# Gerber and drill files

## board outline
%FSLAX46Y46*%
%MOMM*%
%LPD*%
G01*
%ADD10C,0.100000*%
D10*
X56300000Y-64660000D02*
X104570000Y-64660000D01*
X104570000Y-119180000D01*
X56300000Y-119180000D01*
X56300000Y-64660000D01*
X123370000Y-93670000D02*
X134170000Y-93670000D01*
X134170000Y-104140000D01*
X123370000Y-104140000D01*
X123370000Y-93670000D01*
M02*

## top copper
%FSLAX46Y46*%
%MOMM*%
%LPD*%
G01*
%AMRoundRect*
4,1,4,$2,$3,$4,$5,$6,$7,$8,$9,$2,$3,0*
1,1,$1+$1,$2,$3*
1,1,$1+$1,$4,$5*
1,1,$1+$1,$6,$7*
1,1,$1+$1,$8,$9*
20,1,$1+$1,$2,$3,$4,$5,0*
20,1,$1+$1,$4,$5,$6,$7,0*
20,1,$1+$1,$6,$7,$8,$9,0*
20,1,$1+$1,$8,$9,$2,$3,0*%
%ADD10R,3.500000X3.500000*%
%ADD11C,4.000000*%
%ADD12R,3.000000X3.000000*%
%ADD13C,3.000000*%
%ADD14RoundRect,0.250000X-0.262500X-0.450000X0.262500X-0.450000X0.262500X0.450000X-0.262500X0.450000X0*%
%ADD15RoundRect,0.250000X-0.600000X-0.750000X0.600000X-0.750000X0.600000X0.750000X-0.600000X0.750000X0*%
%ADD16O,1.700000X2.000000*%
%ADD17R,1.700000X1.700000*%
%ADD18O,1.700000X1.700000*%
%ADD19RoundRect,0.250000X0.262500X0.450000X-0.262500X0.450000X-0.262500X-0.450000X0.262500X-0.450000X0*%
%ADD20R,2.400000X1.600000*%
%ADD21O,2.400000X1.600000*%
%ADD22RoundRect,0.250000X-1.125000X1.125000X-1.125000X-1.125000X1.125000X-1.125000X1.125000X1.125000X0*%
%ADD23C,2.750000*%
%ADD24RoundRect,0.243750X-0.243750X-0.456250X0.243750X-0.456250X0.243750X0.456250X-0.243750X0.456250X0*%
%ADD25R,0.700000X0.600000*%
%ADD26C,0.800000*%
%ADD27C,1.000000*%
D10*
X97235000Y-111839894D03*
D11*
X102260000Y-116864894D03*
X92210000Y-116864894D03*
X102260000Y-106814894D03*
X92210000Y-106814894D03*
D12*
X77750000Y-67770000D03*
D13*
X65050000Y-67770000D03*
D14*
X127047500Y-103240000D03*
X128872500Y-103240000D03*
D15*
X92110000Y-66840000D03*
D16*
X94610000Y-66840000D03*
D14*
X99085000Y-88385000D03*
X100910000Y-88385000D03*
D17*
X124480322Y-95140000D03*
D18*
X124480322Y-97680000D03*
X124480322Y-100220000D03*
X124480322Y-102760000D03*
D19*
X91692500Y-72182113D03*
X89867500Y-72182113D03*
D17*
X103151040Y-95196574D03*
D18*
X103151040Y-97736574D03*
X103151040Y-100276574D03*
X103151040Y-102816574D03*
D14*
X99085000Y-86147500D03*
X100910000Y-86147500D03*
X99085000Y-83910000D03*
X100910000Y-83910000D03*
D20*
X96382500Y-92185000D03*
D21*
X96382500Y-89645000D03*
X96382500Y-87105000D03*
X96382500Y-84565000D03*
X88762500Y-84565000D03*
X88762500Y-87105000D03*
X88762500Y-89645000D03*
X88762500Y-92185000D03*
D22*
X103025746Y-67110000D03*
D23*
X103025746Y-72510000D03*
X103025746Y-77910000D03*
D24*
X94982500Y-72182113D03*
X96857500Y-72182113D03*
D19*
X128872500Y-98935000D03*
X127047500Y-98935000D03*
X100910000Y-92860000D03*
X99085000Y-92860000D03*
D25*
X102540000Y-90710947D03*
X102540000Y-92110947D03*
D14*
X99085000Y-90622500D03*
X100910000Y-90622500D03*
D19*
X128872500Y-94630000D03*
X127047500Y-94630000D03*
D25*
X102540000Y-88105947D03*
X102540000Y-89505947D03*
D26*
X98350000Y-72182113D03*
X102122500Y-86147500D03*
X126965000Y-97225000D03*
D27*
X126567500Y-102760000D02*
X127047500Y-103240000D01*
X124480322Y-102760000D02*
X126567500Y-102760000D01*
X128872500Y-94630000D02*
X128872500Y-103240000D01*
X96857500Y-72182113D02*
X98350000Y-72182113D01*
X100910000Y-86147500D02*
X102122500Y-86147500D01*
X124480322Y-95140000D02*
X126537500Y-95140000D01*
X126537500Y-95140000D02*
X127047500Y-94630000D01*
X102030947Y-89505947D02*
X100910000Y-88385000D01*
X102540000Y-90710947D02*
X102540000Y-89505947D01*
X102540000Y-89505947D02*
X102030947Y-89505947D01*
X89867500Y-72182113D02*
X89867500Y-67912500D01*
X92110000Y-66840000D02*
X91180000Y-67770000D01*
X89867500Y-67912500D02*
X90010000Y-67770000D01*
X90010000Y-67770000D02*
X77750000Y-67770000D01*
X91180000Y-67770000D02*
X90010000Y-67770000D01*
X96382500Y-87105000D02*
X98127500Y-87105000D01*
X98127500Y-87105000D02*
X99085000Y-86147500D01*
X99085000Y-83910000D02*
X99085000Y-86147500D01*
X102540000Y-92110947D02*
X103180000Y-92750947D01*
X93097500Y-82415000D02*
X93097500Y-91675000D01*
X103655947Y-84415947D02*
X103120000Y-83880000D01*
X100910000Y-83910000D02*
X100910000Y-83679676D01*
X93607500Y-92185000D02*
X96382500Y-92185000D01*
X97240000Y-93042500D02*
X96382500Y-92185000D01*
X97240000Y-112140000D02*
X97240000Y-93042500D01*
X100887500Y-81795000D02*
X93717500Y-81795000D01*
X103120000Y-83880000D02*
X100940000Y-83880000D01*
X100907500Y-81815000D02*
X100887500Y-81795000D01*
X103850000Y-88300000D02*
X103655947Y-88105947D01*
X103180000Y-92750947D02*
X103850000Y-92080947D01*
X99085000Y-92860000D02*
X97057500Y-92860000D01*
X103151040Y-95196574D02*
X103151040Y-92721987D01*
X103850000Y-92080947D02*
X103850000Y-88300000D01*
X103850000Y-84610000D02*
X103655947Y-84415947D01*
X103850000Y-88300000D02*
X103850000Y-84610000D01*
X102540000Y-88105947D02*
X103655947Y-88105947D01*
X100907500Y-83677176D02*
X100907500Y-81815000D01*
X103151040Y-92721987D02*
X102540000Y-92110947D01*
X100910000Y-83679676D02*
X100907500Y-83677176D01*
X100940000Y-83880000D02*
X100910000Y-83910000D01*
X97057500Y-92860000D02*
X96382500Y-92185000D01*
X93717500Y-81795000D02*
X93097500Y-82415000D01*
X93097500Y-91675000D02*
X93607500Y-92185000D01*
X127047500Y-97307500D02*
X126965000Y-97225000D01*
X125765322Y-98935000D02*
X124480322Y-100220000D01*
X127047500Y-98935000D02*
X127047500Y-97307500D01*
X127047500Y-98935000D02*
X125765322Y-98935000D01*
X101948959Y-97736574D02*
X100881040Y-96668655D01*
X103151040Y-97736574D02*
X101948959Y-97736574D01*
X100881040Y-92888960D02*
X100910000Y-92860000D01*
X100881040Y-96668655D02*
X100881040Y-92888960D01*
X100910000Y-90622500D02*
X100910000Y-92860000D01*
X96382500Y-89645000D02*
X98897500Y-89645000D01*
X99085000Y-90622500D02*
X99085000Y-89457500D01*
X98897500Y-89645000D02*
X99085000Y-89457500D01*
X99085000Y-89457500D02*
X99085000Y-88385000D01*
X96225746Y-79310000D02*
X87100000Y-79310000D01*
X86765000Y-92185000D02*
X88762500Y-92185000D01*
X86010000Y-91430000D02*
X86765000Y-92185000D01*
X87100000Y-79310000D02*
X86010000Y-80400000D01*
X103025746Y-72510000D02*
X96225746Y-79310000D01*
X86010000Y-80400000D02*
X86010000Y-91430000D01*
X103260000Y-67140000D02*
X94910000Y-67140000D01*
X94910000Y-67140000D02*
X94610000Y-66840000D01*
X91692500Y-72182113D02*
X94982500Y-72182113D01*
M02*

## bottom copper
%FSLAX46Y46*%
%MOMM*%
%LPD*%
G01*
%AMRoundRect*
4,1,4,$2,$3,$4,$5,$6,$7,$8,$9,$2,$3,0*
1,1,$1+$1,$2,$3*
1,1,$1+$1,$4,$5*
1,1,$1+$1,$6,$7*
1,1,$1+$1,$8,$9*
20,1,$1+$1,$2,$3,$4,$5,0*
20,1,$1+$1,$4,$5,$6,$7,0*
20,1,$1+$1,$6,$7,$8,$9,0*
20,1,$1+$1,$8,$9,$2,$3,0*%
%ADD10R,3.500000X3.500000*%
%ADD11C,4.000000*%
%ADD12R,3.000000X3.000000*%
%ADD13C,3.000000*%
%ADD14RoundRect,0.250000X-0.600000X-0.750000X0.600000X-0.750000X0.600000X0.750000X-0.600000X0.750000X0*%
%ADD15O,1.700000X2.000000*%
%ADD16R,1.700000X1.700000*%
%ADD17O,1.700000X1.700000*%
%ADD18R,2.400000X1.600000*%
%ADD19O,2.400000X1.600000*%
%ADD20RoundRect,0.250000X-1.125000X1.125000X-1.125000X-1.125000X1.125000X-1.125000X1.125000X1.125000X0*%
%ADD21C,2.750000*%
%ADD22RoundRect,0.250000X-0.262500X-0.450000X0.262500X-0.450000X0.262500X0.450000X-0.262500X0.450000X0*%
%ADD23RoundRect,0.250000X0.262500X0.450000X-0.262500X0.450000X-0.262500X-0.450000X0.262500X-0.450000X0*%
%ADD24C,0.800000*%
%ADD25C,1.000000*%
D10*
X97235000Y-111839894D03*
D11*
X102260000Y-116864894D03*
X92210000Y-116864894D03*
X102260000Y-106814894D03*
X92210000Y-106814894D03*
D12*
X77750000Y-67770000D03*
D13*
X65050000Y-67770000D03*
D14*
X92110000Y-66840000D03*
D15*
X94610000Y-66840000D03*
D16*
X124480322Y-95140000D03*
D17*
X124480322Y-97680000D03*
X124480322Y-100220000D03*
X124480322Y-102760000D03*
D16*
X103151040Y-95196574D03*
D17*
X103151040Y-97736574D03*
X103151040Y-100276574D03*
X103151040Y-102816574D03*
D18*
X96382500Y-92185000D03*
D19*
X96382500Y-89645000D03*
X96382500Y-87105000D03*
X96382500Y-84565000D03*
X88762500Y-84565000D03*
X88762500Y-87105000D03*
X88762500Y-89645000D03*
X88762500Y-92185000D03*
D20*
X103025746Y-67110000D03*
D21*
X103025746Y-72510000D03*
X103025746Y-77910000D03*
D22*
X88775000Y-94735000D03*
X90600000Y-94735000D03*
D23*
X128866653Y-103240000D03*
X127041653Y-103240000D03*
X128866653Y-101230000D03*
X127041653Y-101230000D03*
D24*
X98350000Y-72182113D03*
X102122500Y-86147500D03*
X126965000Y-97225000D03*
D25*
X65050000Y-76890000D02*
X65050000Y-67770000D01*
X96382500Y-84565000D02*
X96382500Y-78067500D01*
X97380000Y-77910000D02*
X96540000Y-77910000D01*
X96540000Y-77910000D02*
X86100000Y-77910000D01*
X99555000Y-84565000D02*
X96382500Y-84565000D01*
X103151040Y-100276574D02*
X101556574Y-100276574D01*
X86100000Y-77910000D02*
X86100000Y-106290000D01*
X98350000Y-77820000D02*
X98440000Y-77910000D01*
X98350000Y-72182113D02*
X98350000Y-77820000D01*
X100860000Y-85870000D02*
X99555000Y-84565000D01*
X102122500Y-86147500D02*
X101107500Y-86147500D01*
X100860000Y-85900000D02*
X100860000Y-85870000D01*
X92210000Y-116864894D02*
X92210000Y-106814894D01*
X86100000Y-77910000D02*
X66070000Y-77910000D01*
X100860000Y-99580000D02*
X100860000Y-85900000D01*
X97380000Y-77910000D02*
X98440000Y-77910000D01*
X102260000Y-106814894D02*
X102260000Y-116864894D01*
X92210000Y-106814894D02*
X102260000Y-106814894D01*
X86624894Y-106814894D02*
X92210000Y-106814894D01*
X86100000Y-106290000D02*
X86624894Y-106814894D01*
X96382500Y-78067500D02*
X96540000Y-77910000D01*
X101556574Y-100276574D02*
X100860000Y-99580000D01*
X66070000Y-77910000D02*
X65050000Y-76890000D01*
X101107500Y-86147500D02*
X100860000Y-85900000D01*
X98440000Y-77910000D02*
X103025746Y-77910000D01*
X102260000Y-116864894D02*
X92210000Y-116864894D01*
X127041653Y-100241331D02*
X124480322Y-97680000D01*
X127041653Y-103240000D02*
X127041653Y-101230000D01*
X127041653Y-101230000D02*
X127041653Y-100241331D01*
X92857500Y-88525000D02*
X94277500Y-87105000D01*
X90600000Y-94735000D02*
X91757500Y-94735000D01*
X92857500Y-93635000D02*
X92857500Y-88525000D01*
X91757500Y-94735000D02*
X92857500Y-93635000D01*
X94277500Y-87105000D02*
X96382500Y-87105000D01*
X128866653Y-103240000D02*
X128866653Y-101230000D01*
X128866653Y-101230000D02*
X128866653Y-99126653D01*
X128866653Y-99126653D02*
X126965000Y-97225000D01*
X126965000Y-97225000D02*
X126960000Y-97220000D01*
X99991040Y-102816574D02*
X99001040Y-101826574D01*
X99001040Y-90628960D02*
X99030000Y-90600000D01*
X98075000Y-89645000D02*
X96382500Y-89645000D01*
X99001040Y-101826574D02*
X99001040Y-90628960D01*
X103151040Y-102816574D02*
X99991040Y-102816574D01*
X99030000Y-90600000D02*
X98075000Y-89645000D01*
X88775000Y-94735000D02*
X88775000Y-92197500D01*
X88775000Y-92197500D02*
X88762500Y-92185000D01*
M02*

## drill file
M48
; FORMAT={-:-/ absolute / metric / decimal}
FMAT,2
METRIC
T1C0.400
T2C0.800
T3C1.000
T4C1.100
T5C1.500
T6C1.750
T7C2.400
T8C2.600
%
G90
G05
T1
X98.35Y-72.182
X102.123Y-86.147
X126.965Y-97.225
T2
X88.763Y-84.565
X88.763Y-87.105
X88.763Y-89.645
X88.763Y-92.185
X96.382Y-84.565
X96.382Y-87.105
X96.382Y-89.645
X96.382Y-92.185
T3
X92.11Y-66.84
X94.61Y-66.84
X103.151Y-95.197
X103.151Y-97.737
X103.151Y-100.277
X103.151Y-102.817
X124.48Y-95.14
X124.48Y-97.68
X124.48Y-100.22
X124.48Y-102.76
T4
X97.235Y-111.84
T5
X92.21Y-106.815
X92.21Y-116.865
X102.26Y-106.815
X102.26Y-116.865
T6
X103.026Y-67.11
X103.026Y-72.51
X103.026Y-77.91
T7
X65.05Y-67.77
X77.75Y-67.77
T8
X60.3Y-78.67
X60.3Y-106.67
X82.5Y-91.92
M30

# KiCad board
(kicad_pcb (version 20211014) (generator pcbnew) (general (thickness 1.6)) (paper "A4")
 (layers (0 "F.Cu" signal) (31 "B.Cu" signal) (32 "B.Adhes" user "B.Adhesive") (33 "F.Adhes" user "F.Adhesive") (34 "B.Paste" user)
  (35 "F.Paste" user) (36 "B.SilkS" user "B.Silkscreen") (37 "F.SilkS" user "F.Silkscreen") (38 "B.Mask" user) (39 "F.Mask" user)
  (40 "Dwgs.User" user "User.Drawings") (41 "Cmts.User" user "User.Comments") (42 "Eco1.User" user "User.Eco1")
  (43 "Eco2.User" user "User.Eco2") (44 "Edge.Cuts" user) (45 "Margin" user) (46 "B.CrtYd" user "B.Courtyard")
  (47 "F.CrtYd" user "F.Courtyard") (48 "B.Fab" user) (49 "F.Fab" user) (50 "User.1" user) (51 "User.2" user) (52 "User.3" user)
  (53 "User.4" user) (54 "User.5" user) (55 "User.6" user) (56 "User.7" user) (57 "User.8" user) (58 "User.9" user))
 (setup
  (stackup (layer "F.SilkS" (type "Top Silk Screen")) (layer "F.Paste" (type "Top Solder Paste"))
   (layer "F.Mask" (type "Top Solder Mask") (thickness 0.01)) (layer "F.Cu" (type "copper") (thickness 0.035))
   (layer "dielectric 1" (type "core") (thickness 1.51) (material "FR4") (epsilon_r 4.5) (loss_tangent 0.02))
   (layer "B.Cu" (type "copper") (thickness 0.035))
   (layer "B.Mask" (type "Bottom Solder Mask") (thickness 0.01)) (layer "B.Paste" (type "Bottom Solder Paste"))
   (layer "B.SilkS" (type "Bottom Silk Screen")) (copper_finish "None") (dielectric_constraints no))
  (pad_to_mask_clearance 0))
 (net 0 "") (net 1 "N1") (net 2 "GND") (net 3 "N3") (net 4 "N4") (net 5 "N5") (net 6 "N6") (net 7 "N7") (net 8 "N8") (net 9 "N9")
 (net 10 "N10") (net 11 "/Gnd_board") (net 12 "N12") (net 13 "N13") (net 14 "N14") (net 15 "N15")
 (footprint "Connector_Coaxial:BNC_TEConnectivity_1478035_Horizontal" (layer "F.Cu") (at 97.235 111.839894 -90)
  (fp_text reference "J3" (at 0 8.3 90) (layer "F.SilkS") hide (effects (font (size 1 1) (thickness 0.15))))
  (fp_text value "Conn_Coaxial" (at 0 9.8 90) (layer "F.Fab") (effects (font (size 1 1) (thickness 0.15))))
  (pad "1" thru_hole rect (at 0 0 270) (size 3.5 3.5) (drill 1.1) (layers *.Cu *.Mask) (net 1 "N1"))
  (pad "2" thru_hole circle (at 5.025 -5.025 270) (size 4 4) (drill 1.5) (layers *.Cu *.Mask) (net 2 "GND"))
  (pad "2" thru_hole circle (at 5.025 5.025 270) (size 4 4) (drill 1.5) (layers *.Cu *.Mask) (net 2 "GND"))
  (pad "2" thru_hole circle (at -5.025 -5.025 270) (size 4 4) (drill 1.5) (layers *.Cu *.Mask) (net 2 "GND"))
  (pad "2" thru_hole circle (at -5.025 5.025 270) (size 4 4) (drill 1.5) (layers *.Cu *.Mask) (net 2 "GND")))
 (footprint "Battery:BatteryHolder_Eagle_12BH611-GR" (layer "F.Cu") (at 77.75 67.77 90)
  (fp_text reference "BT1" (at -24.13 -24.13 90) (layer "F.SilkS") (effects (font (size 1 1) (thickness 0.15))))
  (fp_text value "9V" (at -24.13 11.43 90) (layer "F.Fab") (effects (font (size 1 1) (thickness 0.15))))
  (pad "" np_thru_hole circle locked (at -24.15 4.75 90) (size 2.6 2.6) (drill 2.6) (layers *.Cu *.Mask))
  (pad "" np_thru_hole circle locked (at -38.9 -17.45 90) (size 2.6 2.6) (drill 2.6) (layers *.Cu *.Mask))
  (pad "" np_thru_hole circle locked (at -10.9 -17.45 90) (size 2.6 2.6) (drill 2.6) (layers *.Cu *.Mask))
  (pad "1" thru_hole rect locked (at 0 0 90) (size 3 3) (drill 2.4) (layers *.Cu *.Mask) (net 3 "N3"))
  (pad "2" thru_hole circle locked (at 0 -12.7 90) (size 3 3) (drill 2.4) (layers *.Cu *.Mask) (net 2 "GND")))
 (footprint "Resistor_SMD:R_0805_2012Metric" (layer "F.Cu") (at 127.96 103.24)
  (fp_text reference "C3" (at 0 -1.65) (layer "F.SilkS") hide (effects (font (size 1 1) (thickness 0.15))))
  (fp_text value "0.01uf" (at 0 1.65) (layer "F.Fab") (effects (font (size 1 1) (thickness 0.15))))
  (pad "1" smd roundrect locked (at -0.9125 0) (size 1.025 1.4) (layers "F.Cu" "F.Paste" "F.Mask") (roundrect_rratio 0.243902) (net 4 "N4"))
  (pad "2" smd roundrect locked (at 0.9125 0) (size 1.025 1.4) (layers "F.Cu" "F.Paste" "F.Mask") (roundrect_rratio 0.243902) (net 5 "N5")))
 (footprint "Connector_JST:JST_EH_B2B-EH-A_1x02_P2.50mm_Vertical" (layer "F.Cu") (at 92.11 66.84)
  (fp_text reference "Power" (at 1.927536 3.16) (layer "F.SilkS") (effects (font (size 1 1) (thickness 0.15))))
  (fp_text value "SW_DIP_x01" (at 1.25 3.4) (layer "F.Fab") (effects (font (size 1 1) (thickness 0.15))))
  (pad "1" thru_hole roundrect locked (at 0 0) (size 1.7 2) (drill 1) (layers *.Cu *.Mask) (roundrect_rratio 0.147059) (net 3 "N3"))
  (pad "2" thru_hole oval locked (at 2.5 0) (size 1.7 2) (drill 1) (layers *.Cu *.Mask) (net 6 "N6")))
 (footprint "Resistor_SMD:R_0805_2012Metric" (layer "F.Cu") (at 99.9975 88.385)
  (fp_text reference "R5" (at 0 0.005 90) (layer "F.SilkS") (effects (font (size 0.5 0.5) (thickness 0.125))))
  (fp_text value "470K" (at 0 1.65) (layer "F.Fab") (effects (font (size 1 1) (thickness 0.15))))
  (pad "1" smd roundrect locked (at -0.9125 0) (size 1.025 1.4) (layers "F.Cu" "F.Paste" "F.Mask") (roundrect_rratio 0.243902) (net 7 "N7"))
  (pad "2" smd roundrect locked (at 0.9125 0) (size 1.025 1.4) (layers "F.Cu" "F.Paste" "F.Mask") (roundrect_rratio 0.243902) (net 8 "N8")))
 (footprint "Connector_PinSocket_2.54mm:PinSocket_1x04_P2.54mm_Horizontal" (layer "F.Cu") (at 124.480322 95.14)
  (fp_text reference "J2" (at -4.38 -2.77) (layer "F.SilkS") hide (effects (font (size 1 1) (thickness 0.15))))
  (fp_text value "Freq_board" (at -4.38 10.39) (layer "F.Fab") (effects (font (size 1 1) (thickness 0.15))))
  (pad "1" thru_hole rect locked (at 0 0) (size 1.7 1.7) (drill 1) (layers *.Cu *.Mask) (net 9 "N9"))
  (pad "2" thru_hole oval locked (at 0 2.54) (size 1.7 1.7) (drill 1) (layers *.Cu *.Mask) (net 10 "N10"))
  (pad "3" thru_hole oval locked (at 0 5.08) (size 1.7 1.7) (drill 1) (layers *.Cu *.Mask) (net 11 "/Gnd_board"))
  (pad "4" thru_hole oval locked (at 0 7.62) (size 1.7 1.7) (drill 1) (layers *.Cu *.Mask) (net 4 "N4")))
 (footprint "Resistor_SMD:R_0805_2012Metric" (layer "F.Cu") (at 90.78 72.182113 180)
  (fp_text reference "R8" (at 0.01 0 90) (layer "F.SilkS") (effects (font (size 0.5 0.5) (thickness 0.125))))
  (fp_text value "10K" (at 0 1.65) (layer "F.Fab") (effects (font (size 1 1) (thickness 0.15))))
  (pad "1" smd roundrect locked (at -0.9125 0 180) (size 1.025 1.4) (layers "F.Cu" "F.Paste" "F.Mask") (roundrect_rratio 0.243902)
   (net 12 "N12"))
  (pad "2" smd roundrect locked (at 0.9125 0 180) (size 1.025 1.4) (layers "F.Cu" "F.Paste" "F.Mask") (roundrect_rratio 0.243902)
   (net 3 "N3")))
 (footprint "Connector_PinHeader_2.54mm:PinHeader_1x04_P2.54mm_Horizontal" (layer "F.Cu") (at 103.15104 95.196574)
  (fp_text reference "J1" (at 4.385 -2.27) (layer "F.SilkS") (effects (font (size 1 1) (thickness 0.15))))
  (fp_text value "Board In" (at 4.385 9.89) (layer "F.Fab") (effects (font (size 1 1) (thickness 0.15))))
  (pad "1" thru_hole rect locked (at 0 0) (size 1.7 1.7) (drill 1) (layers *.Cu *.Mask) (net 1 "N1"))
  (pad "2" thru_hole oval locked (at 0 2.54) (size 1.7 1.7) (drill 1) (layers *.Cu *.Mask) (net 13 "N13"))
  (pad "3" thru_hole oval locked (at 0 5.08) (size 1.7 1.7) (drill 1) (layers *.Cu *.Mask) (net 2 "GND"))
  (pad "4" thru_hole oval locked (at 0 7.62) (size 1.7 1.7) (drill 1) (layers *.Cu *.Mask) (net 7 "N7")))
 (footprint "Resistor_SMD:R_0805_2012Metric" (layer "F.Cu") (at 99.9975 86.1475)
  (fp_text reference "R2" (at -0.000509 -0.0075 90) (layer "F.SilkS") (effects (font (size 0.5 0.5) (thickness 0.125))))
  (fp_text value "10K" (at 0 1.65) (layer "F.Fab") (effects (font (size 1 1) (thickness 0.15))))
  (pad "1" smd roundrect locked (at -0.9125 0) (size 1.025 1.4) (layers "F.Cu" "F.Paste" "F.Mask") (roundrect_rratio 0.243902)
   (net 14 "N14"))
  (pad "2" smd roundrect locked (at 0.9125 0) (size 1.025 1.4) (layers "F.Cu" "F.Paste" "F.Mask") (roundrect_rratio 0.243902) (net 2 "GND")))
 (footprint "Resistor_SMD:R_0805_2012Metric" (layer "F.Cu") (at 99.9975 83.91)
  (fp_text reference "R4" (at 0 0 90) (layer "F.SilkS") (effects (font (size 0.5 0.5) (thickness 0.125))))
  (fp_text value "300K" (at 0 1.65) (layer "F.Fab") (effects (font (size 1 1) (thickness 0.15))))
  (pad "1" smd roundrect locked (at -0.9125 0) (size 1.025 1.4) (layers "F.Cu" "F.Paste" "F.Mask") (roundrect_rratio 0.243902)
   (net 14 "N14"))
  (pad "2" smd roundrect locked (at 0.9125 0) (size 1.025 1.4) (layers "F.Cu" "F.Paste" "F.Mask") (roundrect_rratio 0.243902) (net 1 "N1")))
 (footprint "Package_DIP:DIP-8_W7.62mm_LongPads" (layer "F.Cu") (at 96.3825 92.185 180)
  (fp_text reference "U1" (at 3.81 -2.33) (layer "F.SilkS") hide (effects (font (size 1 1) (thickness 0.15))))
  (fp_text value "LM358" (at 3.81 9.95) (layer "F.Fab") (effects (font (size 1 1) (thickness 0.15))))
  (pad "1" thru_hole rect locked (at 0 0 180) (size 2.4 1.6) (drill 0.8) (layers *.Cu *.Mask) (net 1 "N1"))
  (pad "2" thru_hole oval locked (at 0 2.54 180) (size 2.4 1.6) (drill 0.8) (layers *.Cu *.Mask) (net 7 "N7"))
  (pad "3" thru_hole oval locked (at 0 5.08 180) (size 2.4 1.6) (drill 0.8) (layers *.Cu *.Mask) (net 14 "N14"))
  (pad "4" thru_hole oval locked (at 0 7.62 180) (size 2.4 1.6) (drill 0.8) (layers *.Cu *.Mask) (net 2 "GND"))
  (pad "5" thru_hole oval locked (at 7.62 7.62 180) (size 2.4 1.6) (drill 0.8) (layers *.Cu *.Mask))
  (pad "6" thru_hole oval locked (at 7.62 5.08 180) (size 2.4 1.6) (drill 0.8) (layers *.Cu *.Mask))
  (pad "7" thru_hole oval locked (at 7.62 2.54 180) (size 2.4 1.6) (drill 0.8) (layers *.Cu *.Mask))
  (pad "8" thru_hole oval locked (at 7.62 0 180) (size 2.4 1.6) (drill 0.8) (layers *.Cu *.Mask) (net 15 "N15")))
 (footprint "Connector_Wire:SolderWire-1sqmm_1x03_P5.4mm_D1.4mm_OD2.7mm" (layer "F.Cu") (at 103.025746 67.11 -90)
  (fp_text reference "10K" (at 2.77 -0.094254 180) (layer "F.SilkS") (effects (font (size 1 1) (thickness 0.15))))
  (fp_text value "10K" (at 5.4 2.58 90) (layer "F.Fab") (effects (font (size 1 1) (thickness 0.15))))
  (pad "1" thru_hole roundrect locked (at 0 0 270) (size 2.75 2.75) (drill 1.75) (layers *.Cu *.Mask) (roundrect_rratio 0.090909)
   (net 6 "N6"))
  (pad "2" thru_hole circle locked (at 5.4 0 270) (size 2.75 2.75) (drill 1.75) (layers *.Cu *.Mask) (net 15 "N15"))
  (pad "3" thru_hole circle locked (at 10.8 0 270) (size 2.75 2.75) (drill 1.75) (layers *.Cu *.Mask) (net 2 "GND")))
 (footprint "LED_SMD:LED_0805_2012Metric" (layer "F.Cu") (at 95.92 72.182113)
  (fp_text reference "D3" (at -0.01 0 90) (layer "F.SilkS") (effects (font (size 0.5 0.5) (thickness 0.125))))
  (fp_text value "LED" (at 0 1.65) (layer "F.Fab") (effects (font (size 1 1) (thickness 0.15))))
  (pad "1" smd roundrect locked (at -0.9375 0) (size 0.975 1.4) (layers "F.Cu" "F.Paste" "F.Mask") (roundrect_rratio 0.25) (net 12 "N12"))
  (pad "2" smd roundrect locked (at 0.9375 0) (size 0.975 1.4) (layers "F.Cu" "F.Paste" "F.Mask") (roundrect_rratio 0.25) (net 2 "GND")))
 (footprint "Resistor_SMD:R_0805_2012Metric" (layer "F.Cu") (at 127.96 98.935 180)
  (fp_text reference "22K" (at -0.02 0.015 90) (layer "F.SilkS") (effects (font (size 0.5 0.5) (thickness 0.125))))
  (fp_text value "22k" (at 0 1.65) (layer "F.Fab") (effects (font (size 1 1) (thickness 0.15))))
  (pad "1" smd roundrect locked (at -0.9125 0 180) (size 1.025 1.4) (layers "F.Cu" "F.Paste" "F.Mask") (roundrect_rratio 0.243902)
   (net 5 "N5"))
  (pad "2" smd roundrect locked (at 0.9125 0 180) (size 1.025 1.4) (layers "F.Cu" "F.Paste" "F.Mask") (roundrect_rratio 0.243902)
   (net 11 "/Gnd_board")))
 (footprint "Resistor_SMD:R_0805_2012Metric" (layer "F.Cu") (at 99.9975 92.86 180)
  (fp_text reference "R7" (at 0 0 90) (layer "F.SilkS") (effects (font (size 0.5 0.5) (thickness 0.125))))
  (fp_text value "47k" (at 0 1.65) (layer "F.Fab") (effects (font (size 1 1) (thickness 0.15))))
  (pad "1" smd roundrect locked (at -0.9125 0 180) (size 1.025 1.4) (layers "F.Cu" "F.Paste" "F.Mask") (roundrect_rratio 0.243902)
   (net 13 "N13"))
  (pad "2" smd roundrect locked (at 0.9125 0 180) (size 1.025 1.4) (layers "F.Cu" "F.Paste" "F.Mask") (roundrect_rratio 0.243902)
   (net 1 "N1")))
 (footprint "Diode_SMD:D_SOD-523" (layer "F.Cu") (at 102.54 91.410947 -90)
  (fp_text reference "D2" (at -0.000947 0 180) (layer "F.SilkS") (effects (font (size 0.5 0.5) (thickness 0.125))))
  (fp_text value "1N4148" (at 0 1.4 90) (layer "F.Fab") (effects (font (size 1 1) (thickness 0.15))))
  (pad "1" smd rect locked (at -0.7 0 90) (size 0.6 0.7) (layers "F.Cu" "F.Paste" "F.Mask") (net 8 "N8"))
  (pad "2" smd rect locked (at 0.7 0 90) (size 0.6 0.7) (layers "F.Cu" "F.Paste" "F.Mask") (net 1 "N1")))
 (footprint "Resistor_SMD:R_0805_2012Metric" (layer "F.Cu") (at 99.9975 90.6225)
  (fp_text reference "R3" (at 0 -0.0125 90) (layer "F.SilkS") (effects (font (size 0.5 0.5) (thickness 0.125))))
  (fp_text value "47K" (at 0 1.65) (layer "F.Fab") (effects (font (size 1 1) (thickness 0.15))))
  (pad "1" smd roundrect locked (at -0.9125 0) (size 1.025 1.4) (layers "F.Cu" "F.Paste" "F.Mask") (roundrect_rratio 0.243902) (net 7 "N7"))
  (pad "2" smd roundrect locked (at 0.9125 0) (size 1.025 1.4) (layers "F.Cu" "F.Paste" "F.Mask") (roundrect_rratio 0.243902) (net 13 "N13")))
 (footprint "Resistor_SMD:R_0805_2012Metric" (layer "F.Cu") (at 127.96 94.63 180)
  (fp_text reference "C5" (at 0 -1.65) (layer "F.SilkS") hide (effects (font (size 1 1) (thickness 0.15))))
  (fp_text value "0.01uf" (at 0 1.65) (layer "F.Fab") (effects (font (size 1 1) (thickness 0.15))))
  (pad "1" smd roundrect locked (at -0.9125 0 180) (size 1.025 1.4) (layers "F.Cu" "F.Paste" "F.Mask") (roundrect_rratio 0.243902)
   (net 5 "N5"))
  (pad "2" smd roundrect locked (at 0.9125 0 180) (size 1.025 1.4) (layers "F.Cu" "F.Paste" "F.Mask") (roundrect_rratio 0.243902)
   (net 9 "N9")))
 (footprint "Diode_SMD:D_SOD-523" (layer "F.Cu") (at 102.54 88.805947 -90)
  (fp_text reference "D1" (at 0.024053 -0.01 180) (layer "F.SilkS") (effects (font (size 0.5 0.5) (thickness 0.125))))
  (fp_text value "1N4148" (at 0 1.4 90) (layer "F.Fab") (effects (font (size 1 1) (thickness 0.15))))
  (pad "1" smd rect locked (at -0.7 0 90) (size 0.6 0.7) (layers "F.Cu" "F.Paste" "F.Mask") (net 1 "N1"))
  (pad "2" smd rect locked (at 0.7 0 90) (size 0.6 0.7) (layers "F.Cu" "F.Paste" "F.Mask") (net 8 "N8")))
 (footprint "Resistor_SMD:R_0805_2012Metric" (layer "B.Cu") (at 89.6875 94.735)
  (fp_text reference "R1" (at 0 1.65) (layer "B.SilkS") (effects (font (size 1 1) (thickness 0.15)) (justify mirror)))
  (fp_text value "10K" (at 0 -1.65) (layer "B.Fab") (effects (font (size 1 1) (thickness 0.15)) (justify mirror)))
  (pad "1" smd roundrect locked (at -0.9125 0) (size 1.025 1.4) (layers "B.Cu" "B.Paste" "B.Mask") (roundrect_rratio 0.243902)
   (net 15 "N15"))
  (pad "2" smd roundrect locked (at 0.9125 0) (size 1.025 1.4) (layers "B.Cu" "B.Paste" "B.Mask") (roundrect_rratio 0.243902) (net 14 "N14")))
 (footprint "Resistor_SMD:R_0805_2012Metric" (layer "B.Cu") (at 127.954153 103.24 180)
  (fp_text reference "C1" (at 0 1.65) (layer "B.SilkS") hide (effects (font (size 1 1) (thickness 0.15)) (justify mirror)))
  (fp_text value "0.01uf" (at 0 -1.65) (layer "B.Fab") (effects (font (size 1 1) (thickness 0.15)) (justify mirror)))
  (pad "1" smd roundrect locked (at -0.9125 0 180) (size 1.025 1.4) (layers "B.Cu" "B.Paste" "B.Mask") (roundrect_rratio 0.243902)
   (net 11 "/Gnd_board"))
  (pad "2" smd roundrect locked (at 0.9125 0 180) (size 1.025 1.4) (layers "B.Cu" "B.Paste" "B.Mask") (roundrect_rratio 0.243902)
   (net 10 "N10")))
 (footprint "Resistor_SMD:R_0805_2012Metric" (layer "B.Cu") (at 127.954153 101.23 180)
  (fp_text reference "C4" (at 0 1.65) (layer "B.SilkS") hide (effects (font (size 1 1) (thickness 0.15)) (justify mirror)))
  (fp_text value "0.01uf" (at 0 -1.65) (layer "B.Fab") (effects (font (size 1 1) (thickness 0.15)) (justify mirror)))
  (pad "1" smd roundrect locked (at -0.9125 0 180) (size 1.025 1.4) (layers "B.Cu" "B.Paste" "B.Mask") (roundrect_rratio 0.243902)
   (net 11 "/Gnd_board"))
  (pad "2" smd roundrect locked (at 0.9125 0 180) (size 1.025 1.4) (layers "B.Cu" "B.Paste" "B.Mask") (roundrect_rratio 0.243902)
   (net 10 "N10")))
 (gr_rect (start 56.3 64.66) (end 104.57 119.18) (layer "Edge.Cuts") (width 0.1) (fill none))
 (gr_rect (start 123.37 93.67) (end 134.17 104.14) (layer "Edge.Cuts") (width 0.1) (fill none))
 (segment (start 126.5675 102.76) (end 127.0475 103.24) (width 1) (layer "F.Cu") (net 4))
 (segment (start 124.480322 102.76) (end 126.5675 102.76) (width 1) (layer "F.Cu") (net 4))
 (segment (start 128.8725 94.63) (end 128.8725 103.24) (width 1) (layer "F.Cu") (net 5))
 (segment (start 96.8575 72.182113) (end 98.35 72.182113) (width 1) (layer "F.Cu") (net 2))
 (segment (start 100.91 86.1475) (end 102.1225 86.1475) (width 1) (layer "F.Cu") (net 2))
 (via (at 98.35 72.182113) (size 0.8) (drill 0.4) (layers "F.Cu" "B.Cu") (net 2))
 (via (at 102.1225 86.1475) (size 0.8) (drill 0.4) (layers "F.Cu" "B.Cu") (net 2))
 (segment (start 65.05 76.89) (end 65.05 67.77) (width 1) (layer "B.Cu") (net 2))
 (segment (start 96.3825 84.565) (end 96.3825 78.0675) (width 1) (layer "B.Cu") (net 2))
 (segment (start 97.38 77.91) (end 96.54 77.91) (width 1) (layer "B.Cu") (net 2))
 (segment (start 96.54 77.91) (end 86.1 77.91) (width 1) (layer "B.Cu") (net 2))
 (segment (start 99.555 84.565) (end 96.3825 84.565) (width 1) (layer "B.Cu") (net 2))
 (segment (start 103.15104 100.276574) (end 101.556574 100.276574) (width 1) (layer "B.Cu") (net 2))
 (segment (start 86.1 77.91) (end 86.1 106.29) (width 1) (layer "B.Cu") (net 2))
 (segment (start 98.35 77.82) (end 98.44 77.91) (width 1) (layer "B.Cu") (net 2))
 (segment (start 98.35 72.182113) (end 98.35 77.82) (width 1) (layer "B.Cu") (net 2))
 (segment (start 100.86 85.87) (end 99.555 84.565) (width 1) (layer "B.Cu") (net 2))
 (segment (start 102.1225 86.1475) (end 101.1075 86.1475) (width 1) (layer "B.Cu") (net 2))
 (segment (start 100.86 85.9) (end 100.86 85.87) (width 1) (layer "B.Cu") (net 2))
 (segment (start 92.21 116.864894) (end 92.21 106.814894) (width 1) (layer "B.Cu") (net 2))
 (segment (start 86.1 77.91) (end 66.07 77.91) (width 1) (layer "B.Cu") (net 2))
 (segment (start 100.86 99.58) (end 100.86 85.9) (width 1) (layer "B.Cu") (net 2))
 (segment (start 97.38 77.91) (end 98.44 77.91) (width 1) (layer "B.Cu") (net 2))
 (segment (start 102.26 106.814894) (end 102.26 116.864894) (width 1) (layer "B.Cu") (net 2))
 (segment (start 92.21 106.814894) (end 102.26 106.814894) (width 1) (layer "B.Cu") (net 2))
 (segment (start 86.624894 106.814894) (end 92.21 106.814894) (width 1) (layer "B.Cu") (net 2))
 (segment (start 86.1 106.29) (end 86.624894 106.814894) (width 1) (layer "B.Cu") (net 2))
 (segment (start 96.3825 78.0675) (end 96.54 77.91) (width 1) (layer "B.Cu") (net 2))
 (segment (start 101.556574 100.276574) (end 100.86 99.58) (width 1) (layer "B.Cu") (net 2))
 (segment (start 66.07 77.91) (end 65.05 76.89) (width 1) (layer "B.Cu") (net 2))
 (segment (start 101.1075 86.1475) (end 100.86 85.9) (width 1) (layer "B.Cu") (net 2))
 (segment (start 98.44 77.91) (end 103.025746 77.91) (width 1) (layer "B.Cu") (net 2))
 (segment (start 102.26 116.864894) (end 92.21 116.864894) (width 1) (layer "B.Cu") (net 2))
 (segment (start 127.041653 100.241331) (end 124.480322 97.68) (width 1) (layer "B.Cu") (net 10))
 (segment (start 127.041653 103.24) (end 127.041653 101.23) (width 1) (layer "B.Cu") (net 10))
 (segment (start 127.041653 101.23) (end 127.041653 100.241331) (width 1) (layer "B.Cu") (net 10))
 (segment (start 124.480322 95.14) (end 126.5375 95.14) (width 1) (layer "F.Cu") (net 9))
 (segment (start 126.5375 95.14) (end 127.0475 94.63) (width 1) (layer "F.Cu") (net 9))
 (segment (start 102.030947 89.505947) (end 100.91 88.385) (width 1) (layer "F.Cu") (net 8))
 (segment (start 102.54 90.710947) (end 102.54 89.505947) (width 1) (layer "F.Cu") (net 8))
 (segment (start 102.54 89.505947) (end 102.030947 89.505947) (width 1) (layer "F.Cu") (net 8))
 (segment (start 89.8675 72.182113) (end 89.8675 67.9125) (width 1) (layer "F.Cu") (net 3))
 (segment (start 92.11 66.84) (end 91.18 67.77) (width 1) (layer "F.Cu") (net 3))
 (segment (start 89.8675 67.9125) (end 90.01 67.77) (width 1) (layer "F.Cu") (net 3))
 (segment (start 90.01 67.77) (end 77.75 67.77) (width 1) (layer "F.Cu") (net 3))
 (segment (start 91.18 67.77) (end 90.01 67.77) (width 1) (layer "F.Cu") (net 3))
 (segment (start 96.3825 87.105) (end 98.1275 87.105) (width 1) (layer "F.Cu") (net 14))
 (segment (start 98.1275 87.105) (end 99.085 86.1475) (width 1) (layer "F.Cu") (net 14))
 (segment (start 99.085 83.91) (end 99.085 86.1475) (width 1) (layer "F.Cu") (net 14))
 (segment (start 92.8575 88.525) (end 94.2775 87.105) (width 1) (layer "B.Cu") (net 14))
 (segment (start 90.6 94.735) (end 91.7575 94.735) (width 1) (layer "B.Cu") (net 14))
 (segment (start 92.8575 93.635) (end 92.8575 88.525) (width 1) (layer "B.Cu") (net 14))
 (segment (start 91.7575 94.735) (end 92.8575 93.635) (width 1) (layer "B.Cu") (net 14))
 (segment (start 94.2775 87.105) (end 96.3825 87.105) (width 1) (layer "B.Cu") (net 14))
 (segment (start 102.54 92.110947) (end 103.18 92.750947) (width 1) (layer "F.Cu") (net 1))
 (segment (start 93.0975 82.415) (end 93.0975 91.675) (width 1) (layer "F.Cu") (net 1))
 (segment (start 103.655947 84.415947) (end 103.12 83.88) (width 1) (layer "F.Cu") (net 1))
 (segment (start 100.91 83.91) (end 100.91 83.679676) (width 1) (layer "F.Cu") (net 1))
 (segment (start 93.6075 92.185) (end 96.3825 92.185) (width 1) (layer "F.Cu") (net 1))
 (segment (start 97.24 93.0425) (end 96.3825 92.185) (width 1) (layer "F.Cu") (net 1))
 (segment (start 97.24 112.14) (end 97.24 93.0425) (width 1) (layer "F.Cu") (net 1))
 (segment (start 100.8875 81.795) (end 93.7175 81.795) (width 1) (layer "F.Cu") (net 1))
 (segment (start 103.12 83.88) (end 100.94 83.88) (width 1) (layer "F.Cu") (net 1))
 (segment (start 100.9075 81.815) (end 100.8875 81.795) (width 1) (layer "F.Cu") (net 1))
 (segment (start 103.85 88.3) (end 103.655947 88.105947) (width 1) (layer "F.Cu") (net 1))
 (segment (start 103.18 92.750947) (end 103.85 92.080947) (width 1) (layer "F.Cu") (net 1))
 (segment (start 99.085 92.86) (end 97.0575 92.86) (width 1) (layer "F.Cu") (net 1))
 (segment (start 103.15104 95.196574) (end 103.15104 92.721987) (width 1) (layer "F.Cu") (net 1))
 (segment (start 103.85 92.080947) (end 103.85 88.3) (width 1) (layer "F.Cu") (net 1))
 (segment (start 103.85 84.61) (end 103.655947 84.415947) (width 1) (layer "F.Cu") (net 1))
 (segment (start 103.85 88.3) (end 103.85 84.61) (width 1) (layer "F.Cu") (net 1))
 (segment (start 102.54 88.105947) (end 103.655947 88.105947) (width 1) (layer "F.Cu") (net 1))
 (segment (start 100.9075 83.677176) (end 100.9075 81.815) (width 1) (layer "F.Cu") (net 1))
 (segment (start 103.15104 92.721987) (end 102.54 92.110947) (width 1) (layer "F.Cu") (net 1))
 (segment (start 100.91 83.679676) (end 100.9075 83.677176) (width 1) (layer "F.Cu") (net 1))
 (segment (start 100.94 83.88) (end 100.91 83.91) (width 1) (layer "F.Cu") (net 1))
 (segment (start 97.0575 92.86) (end 96.3825 92.185) (width 1) (layer "F.Cu") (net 1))
 (segment (start 93.7175 81.795) (end 93.0975 82.415) (width 1) (layer "F.Cu") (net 1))
 (segment (start 93.0975 91.675) (end 93.6075 92.185) (width 1) (layer "F.Cu") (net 1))
 (segment (start 127.0475 97.3075) (end 126.965 97.225) (width 1) (layer "F.Cu") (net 11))
 (segment (start 125.765322 98.935) (end 124.480322 100.22) (width 1) (layer "F.Cu") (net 11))
 (segment (start 127.0475 98.935) (end 127.0475 97.3075) (width 1) (layer "F.Cu") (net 11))
 (segment (start 127.0475 98.935) (end 125.765322 98.935) (width 1) (layer "F.Cu") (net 11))
 (via (at 126.965 97.225) (size 0.8) (drill 0.4) (layers "F.Cu" "B.Cu") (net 11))
 (segment (start 128.866653 103.24) (end 128.866653 101.23) (width 1) (layer "B.Cu") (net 11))
 (segment (start 128.866653 101.23) (end 128.866653 99.126653) (width 1) (layer "B.Cu") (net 11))
 (segment (start 128.866653 99.126653) (end 126.965 97.225) (width 1) (layer "B.Cu") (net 11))
 (segment (start 126.965 97.225) (end 126.96 97.22) (width 1) (layer "B.Cu") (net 11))
 (segment (start 101.948959 97.736574) (end 100.88104 96.668655) (width 1) (layer "F.Cu") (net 13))
 (segment (start 103.15104 97.736574) (end 101.948959 97.736574) (width 1) (layer "F.Cu") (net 13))
 (segment (start 100.88104 92.88896) (end 100.91 92.86) (width 1) (layer "F.Cu") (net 13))
 (segment (start 100.88104 96.668655) (end 100.88104 92.88896) (width 1) (layer "F.Cu") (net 13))
 (segment (start 100.91 90.6225) (end 100.91 92.86) (width 1) (layer "F.Cu") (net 13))
 (segment (start 96.3825 89.645) (end 98.8975 89.645) (width 1) (layer "F.Cu") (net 7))
 (segment (start 99.085 90.6225) (end 99.085 89.4575) (width 1) (layer "F.Cu") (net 7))
 (segment (start 98.8975 89.645) (end 99.085 89.4575) (width 1) (layer "F.Cu") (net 7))
 (segment (start 99.085 89.4575) (end 99.085 88.385) (width 1) (layer "F.Cu") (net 7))
 (segment (start 99.99104 102.816574) (end 99.00104 101.826574) (width 1) (layer "B.Cu") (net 7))
 (segment (start 99.00104 90.62896) (end 99.03 90.6) (width 1) (layer "B.Cu") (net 7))
 (segment (start 98.075 89.645) (end 96.3825 89.645) (width 1) (layer "B.Cu") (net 7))
 (segment (start 99.00104 101.826574) (end 99.00104 90.62896) (width 1) (layer "B.Cu") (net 7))
 (segment (start 103.15104 102.816574) (end 99.99104 102.816574) (width 1) (layer "B.Cu") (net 7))
 (segment (start 99.03 90.6) (end 98.075 89.645) (width 1) (layer "B.Cu") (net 7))
 (segment (start 96.225746 79.31) (end 87.1 79.31) (width 1) (layer "F.Cu") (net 15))
 (segment (start 86.765 92.185) (end 88.7625 92.185) (width 1) (layer "F.Cu") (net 15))
 (segment (start 86.01 91.43) (end 86.765 92.185) (width 1) (layer "F.Cu") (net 15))
 (segment (start 87.1 79.31) (end 86.01 80.4) (width 1) (layer "F.Cu") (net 15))
 (segment (start 103.025746 72.51) (end 96.225746 79.31) (width 1) (layer "F.Cu") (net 15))
 (segment (start 86.01 80.4) (end 86.01 91.43) (width 1) (layer "F.Cu") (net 15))
 (segment (start 88.775 94.735) (end 88.775 92.1975) (width 1) (layer "B.Cu") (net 15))
 (segment (start 88.775 92.1975) (end 88.7625 92.185) (width 1) (layer "B.Cu") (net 15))
 (segment (start 103.26 67.14) (end 94.91 67.14) (width 1) (layer "F.Cu") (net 6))
 (segment (start 94.91 67.14) (end 94.61 66.84) (width 1) (layer "F.Cu") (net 6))
 (segment (start 91.6925 72.182113) (end 94.9825 72.182113) (width 1) (layer "F.Cu") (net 12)))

